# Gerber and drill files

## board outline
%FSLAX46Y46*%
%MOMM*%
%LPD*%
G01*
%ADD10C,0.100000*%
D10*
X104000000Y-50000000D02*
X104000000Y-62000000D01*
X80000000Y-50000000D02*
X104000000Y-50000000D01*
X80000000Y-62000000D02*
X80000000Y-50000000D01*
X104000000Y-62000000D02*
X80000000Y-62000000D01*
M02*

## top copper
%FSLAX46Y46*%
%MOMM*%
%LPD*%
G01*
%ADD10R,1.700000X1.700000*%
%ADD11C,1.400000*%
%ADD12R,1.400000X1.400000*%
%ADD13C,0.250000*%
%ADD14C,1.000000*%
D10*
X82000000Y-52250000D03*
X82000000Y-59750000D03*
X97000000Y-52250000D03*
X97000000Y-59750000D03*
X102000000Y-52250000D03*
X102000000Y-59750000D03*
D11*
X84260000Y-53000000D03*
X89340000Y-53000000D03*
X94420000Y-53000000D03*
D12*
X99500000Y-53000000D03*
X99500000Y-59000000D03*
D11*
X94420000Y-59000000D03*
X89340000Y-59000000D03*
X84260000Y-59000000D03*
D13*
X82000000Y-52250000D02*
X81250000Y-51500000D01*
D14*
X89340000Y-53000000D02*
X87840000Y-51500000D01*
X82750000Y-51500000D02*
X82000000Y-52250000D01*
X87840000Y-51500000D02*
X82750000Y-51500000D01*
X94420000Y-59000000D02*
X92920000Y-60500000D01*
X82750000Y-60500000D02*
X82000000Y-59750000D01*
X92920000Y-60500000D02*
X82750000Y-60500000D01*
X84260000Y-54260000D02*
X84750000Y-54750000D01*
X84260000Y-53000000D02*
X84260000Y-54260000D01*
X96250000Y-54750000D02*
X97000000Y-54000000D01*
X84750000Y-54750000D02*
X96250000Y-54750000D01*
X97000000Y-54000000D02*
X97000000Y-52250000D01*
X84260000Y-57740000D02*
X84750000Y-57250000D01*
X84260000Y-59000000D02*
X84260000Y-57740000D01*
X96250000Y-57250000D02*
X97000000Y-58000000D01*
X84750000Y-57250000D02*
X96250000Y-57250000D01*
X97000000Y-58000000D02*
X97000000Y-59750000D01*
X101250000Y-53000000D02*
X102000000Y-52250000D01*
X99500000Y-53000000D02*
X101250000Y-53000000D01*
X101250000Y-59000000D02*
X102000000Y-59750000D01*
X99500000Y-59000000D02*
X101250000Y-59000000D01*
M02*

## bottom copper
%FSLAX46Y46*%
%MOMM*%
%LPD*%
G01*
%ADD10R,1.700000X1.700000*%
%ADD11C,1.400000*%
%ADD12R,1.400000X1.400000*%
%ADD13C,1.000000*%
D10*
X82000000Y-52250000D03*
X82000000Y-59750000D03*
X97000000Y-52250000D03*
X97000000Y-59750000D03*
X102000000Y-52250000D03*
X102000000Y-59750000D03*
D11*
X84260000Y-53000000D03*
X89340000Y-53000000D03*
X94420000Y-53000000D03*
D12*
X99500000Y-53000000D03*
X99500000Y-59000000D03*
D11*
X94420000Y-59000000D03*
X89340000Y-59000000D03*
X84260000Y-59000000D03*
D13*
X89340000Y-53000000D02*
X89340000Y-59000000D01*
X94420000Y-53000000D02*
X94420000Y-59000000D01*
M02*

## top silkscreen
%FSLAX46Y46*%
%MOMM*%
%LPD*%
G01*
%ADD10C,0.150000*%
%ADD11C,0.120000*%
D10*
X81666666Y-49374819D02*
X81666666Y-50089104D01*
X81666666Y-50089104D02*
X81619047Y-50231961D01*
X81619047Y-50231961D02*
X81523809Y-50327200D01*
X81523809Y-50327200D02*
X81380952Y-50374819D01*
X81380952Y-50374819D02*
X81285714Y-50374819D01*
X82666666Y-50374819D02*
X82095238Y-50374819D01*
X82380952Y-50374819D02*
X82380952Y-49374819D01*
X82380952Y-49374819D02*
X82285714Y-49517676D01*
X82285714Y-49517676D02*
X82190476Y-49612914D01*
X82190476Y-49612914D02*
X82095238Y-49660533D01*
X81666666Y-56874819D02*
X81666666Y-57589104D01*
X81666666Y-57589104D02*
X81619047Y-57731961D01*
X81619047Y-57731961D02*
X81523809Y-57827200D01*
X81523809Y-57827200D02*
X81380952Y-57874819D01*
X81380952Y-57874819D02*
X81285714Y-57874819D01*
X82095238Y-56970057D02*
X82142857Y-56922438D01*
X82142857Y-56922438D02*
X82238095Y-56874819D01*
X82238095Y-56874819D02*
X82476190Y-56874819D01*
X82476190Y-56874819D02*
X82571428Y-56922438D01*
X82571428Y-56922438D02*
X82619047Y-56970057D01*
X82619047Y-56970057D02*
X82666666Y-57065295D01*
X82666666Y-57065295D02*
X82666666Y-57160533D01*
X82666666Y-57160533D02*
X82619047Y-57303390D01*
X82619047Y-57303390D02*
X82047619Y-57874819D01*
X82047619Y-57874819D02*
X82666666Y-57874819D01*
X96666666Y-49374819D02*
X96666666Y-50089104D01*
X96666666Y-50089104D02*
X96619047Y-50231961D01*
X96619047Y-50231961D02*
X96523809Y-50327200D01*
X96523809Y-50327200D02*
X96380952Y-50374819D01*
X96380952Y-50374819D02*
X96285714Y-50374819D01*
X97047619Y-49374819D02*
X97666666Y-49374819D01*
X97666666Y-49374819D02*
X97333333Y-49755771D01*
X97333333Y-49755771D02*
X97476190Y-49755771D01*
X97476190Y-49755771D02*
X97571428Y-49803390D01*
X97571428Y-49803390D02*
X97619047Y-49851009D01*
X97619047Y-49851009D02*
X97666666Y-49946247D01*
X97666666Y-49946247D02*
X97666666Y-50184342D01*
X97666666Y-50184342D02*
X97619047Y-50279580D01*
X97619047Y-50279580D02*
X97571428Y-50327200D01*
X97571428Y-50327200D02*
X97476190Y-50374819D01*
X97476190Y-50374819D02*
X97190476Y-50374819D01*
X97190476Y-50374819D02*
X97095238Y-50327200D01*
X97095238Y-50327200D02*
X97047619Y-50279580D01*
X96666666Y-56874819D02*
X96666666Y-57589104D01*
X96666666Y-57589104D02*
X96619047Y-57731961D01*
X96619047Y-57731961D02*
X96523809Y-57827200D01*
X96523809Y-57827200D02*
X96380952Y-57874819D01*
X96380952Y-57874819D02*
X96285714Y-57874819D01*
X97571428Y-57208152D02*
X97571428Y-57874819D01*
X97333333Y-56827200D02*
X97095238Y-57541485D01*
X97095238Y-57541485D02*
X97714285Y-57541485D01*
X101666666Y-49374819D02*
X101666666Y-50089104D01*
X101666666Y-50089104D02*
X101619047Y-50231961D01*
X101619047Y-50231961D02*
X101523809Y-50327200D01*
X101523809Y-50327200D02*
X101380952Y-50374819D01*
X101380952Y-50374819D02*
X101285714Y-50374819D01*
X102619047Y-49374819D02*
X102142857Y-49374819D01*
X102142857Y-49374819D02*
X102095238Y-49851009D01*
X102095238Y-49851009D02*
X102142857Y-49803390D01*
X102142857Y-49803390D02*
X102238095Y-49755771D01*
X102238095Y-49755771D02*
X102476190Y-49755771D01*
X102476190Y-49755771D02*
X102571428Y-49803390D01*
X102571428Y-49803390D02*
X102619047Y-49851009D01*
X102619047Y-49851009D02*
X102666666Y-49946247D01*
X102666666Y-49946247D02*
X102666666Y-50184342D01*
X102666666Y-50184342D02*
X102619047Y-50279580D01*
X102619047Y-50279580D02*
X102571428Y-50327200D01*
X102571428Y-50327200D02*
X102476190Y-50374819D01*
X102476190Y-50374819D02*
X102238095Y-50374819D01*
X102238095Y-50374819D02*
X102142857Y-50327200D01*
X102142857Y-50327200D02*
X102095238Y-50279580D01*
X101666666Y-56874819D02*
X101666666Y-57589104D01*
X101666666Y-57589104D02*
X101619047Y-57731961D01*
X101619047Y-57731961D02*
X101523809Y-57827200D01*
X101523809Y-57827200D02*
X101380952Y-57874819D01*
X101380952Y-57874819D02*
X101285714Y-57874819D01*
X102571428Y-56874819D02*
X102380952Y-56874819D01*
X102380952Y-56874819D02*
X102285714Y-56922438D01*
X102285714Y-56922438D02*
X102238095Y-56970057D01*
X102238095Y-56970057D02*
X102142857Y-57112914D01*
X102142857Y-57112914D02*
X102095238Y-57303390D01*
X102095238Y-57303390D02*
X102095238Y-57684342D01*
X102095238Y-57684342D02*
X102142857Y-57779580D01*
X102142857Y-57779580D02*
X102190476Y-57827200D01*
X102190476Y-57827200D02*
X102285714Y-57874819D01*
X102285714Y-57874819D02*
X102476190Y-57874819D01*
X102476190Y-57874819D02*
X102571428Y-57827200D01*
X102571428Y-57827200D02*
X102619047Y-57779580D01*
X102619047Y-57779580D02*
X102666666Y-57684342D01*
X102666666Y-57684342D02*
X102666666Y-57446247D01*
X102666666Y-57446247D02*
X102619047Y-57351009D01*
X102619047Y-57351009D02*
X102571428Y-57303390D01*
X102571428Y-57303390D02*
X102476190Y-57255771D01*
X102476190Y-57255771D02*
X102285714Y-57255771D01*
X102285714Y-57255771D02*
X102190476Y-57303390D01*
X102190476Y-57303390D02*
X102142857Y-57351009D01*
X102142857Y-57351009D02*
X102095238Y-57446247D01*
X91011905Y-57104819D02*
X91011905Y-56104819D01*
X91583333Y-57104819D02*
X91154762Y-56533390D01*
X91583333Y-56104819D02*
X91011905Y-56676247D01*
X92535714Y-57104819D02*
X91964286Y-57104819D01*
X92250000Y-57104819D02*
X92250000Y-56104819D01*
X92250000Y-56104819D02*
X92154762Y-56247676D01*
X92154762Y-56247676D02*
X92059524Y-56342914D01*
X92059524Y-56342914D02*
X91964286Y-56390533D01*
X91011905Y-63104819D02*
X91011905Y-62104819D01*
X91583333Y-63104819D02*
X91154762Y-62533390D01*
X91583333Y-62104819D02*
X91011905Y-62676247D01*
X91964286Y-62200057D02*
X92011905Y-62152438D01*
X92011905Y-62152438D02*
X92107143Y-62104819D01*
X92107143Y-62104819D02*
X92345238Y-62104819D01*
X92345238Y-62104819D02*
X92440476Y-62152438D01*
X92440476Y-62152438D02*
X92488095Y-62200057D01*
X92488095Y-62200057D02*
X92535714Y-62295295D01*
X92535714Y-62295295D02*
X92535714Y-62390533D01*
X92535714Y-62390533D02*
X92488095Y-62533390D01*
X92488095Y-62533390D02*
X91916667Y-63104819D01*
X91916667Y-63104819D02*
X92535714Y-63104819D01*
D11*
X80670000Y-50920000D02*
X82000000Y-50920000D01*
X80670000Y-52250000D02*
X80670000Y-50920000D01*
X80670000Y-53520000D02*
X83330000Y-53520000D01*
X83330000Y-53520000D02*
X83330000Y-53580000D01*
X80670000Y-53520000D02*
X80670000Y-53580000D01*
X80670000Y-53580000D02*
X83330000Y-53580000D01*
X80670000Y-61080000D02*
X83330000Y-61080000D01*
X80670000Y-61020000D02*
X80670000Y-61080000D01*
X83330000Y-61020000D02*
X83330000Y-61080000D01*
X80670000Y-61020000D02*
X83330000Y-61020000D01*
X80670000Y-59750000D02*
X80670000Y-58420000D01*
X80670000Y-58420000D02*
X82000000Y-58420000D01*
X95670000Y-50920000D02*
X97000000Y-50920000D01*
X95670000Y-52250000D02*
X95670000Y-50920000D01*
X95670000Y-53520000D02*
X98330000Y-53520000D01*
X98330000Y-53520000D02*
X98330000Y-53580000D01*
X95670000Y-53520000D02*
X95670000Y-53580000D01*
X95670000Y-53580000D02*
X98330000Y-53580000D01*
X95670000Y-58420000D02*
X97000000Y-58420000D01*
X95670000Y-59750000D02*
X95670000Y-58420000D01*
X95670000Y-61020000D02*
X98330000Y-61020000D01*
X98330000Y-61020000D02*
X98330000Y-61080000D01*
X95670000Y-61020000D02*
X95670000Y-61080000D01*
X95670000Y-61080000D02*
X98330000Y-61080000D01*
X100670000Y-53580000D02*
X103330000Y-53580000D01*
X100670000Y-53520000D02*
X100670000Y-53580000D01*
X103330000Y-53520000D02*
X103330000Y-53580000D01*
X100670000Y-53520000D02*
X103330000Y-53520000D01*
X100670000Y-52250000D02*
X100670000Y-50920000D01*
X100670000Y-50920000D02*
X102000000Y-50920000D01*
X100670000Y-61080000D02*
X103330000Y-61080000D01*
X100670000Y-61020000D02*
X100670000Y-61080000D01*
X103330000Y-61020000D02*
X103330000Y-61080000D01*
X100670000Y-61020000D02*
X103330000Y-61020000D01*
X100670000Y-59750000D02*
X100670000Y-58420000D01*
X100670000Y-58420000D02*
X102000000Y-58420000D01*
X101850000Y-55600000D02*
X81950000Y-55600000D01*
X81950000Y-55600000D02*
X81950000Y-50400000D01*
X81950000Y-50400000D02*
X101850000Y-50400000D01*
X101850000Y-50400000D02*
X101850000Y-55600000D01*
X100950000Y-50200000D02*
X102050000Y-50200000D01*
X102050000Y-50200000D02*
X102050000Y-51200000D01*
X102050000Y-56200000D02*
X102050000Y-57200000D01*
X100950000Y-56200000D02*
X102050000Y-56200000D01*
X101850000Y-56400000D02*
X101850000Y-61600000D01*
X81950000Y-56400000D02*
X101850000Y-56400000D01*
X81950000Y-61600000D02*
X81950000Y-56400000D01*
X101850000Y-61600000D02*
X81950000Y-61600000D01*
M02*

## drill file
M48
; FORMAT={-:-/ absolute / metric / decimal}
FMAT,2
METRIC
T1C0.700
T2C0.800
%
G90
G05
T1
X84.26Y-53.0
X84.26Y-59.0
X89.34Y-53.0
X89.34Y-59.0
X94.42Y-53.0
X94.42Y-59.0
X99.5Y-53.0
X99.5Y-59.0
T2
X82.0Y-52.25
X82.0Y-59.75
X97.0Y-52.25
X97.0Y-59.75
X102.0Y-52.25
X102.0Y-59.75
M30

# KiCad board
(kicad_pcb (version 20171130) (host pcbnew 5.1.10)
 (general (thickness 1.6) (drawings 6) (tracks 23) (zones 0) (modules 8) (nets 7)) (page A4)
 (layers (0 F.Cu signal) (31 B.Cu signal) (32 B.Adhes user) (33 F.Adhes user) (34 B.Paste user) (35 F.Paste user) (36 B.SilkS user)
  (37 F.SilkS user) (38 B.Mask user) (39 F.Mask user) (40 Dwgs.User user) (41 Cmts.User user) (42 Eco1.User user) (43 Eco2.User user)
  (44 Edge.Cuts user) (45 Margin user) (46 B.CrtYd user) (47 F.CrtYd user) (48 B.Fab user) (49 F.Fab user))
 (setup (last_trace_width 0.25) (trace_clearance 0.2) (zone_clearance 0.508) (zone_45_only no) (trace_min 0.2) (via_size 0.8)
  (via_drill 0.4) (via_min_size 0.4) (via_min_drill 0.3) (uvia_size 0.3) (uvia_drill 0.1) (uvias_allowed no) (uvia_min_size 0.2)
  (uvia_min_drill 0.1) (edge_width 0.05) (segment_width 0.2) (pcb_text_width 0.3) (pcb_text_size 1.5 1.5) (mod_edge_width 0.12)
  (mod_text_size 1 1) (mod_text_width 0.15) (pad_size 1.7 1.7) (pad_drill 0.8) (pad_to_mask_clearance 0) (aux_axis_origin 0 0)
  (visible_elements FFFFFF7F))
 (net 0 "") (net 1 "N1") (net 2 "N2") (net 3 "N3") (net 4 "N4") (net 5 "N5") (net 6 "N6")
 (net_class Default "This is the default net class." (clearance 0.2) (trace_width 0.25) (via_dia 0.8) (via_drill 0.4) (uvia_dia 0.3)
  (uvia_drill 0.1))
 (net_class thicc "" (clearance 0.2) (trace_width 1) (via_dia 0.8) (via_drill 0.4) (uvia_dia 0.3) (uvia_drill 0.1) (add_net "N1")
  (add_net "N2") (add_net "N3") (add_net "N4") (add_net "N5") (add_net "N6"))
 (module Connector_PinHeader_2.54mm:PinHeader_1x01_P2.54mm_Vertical (layer F.Cu) (at 82 52.25)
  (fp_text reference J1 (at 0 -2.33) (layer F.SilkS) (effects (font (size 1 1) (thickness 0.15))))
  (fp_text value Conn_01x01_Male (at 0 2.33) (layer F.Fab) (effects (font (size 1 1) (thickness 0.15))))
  (fp_line (start -1.33 -1.33) (end 0 -1.33) (layer F.SilkS) (width 0.12))
  (fp_line (start -1.33 0) (end -1.33 -1.33) (layer F.SilkS) (width 0.12))
  (fp_line (start -1.33 1.27) (end 1.33 1.27) (layer F.SilkS) (width 0.12))
  (fp_line (start 1.33 1.27) (end 1.33 1.33) (layer F.SilkS) (width 0.12))
  (fp_line (start -1.33 1.27) (end -1.33 1.33) (layer F.SilkS) (width 0.12))
  (fp_line (start -1.33 1.33) (end 1.33 1.33) (layer F.SilkS) (width 0.12))
  (pad 1 thru_hole rect (at 0 0) (size 1.7 1.7) (drill 0.8) (layers *.Cu *.Mask) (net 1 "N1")))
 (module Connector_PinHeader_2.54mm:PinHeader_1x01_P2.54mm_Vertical (layer F.Cu) (at 82 59.75)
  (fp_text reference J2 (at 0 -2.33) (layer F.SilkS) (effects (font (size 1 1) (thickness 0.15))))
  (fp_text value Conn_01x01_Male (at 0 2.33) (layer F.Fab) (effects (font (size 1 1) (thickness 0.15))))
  (fp_line (start -1.33 1.33) (end 1.33 1.33) (layer F.SilkS) (width 0.12))
  (fp_line (start -1.33 1.27) (end -1.33 1.33) (layer F.SilkS) (width 0.12))
  (fp_line (start 1.33 1.27) (end 1.33 1.33) (layer F.SilkS) (width 0.12))
  (fp_line (start -1.33 1.27) (end 1.33 1.27) (layer F.SilkS) (width 0.12))
  (fp_line (start -1.33 0) (end -1.33 -1.33) (layer F.SilkS) (width 0.12))
  (fp_line (start -1.33 -1.33) (end 0 -1.33) (layer F.SilkS) (width 0.12))
  (pad 1 thru_hole rect (at 0 0) (size 1.7 1.7) (drill 0.8) (layers *.Cu *.Mask) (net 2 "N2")))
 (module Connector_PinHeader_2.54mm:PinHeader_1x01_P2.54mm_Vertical (layer F.Cu) (at 97 52.25)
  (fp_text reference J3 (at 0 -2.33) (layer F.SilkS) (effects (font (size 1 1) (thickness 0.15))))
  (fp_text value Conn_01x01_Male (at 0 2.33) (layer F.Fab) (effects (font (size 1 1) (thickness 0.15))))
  (fp_line (start -1.33 -1.33) (end 0 -1.33) (layer F.SilkS) (width 0.12))
  (fp_line (start -1.33 0) (end -1.33 -1.33) (layer F.SilkS) (width 0.12))
  (fp_line (start -1.33 1.27) (end 1.33 1.27) (layer F.SilkS) (width 0.12))
  (fp_line (start 1.33 1.27) (end 1.33 1.33) (layer F.SilkS) (width 0.12))
  (fp_line (start -1.33 1.27) (end -1.33 1.33) (layer F.SilkS) (width 0.12))
  (fp_line (start -1.33 1.33) (end 1.33 1.33) (layer F.SilkS) (width 0.12))
  (pad 1 thru_hole rect (at 0 0) (size 1.7 1.7) (drill 0.8) (layers *.Cu *.Mask) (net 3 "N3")))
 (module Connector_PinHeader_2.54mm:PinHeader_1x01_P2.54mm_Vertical (layer F.Cu) (at 97 59.75)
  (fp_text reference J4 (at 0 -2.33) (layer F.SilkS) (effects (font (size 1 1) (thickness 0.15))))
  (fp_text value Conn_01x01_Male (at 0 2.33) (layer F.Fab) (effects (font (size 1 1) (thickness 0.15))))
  (fp_line (start -1.33 -1.33) (end 0 -1.33) (layer F.SilkS) (width 0.12))
  (fp_line (start -1.33 0) (end -1.33 -1.33) (layer F.SilkS) (width 0.12))
  (fp_line (start -1.33 1.27) (end 1.33 1.27) (layer F.SilkS) (width 0.12))
  (fp_line (start 1.33 1.27) (end 1.33 1.33) (layer F.SilkS) (width 0.12))
  (fp_line (start -1.33 1.27) (end -1.33 1.33) (layer F.SilkS) (width 0.12))
  (fp_line (start -1.33 1.33) (end 1.33 1.33) (layer F.SilkS) (width 0.12))
  (pad 1 thru_hole rect (at 0 0) (size 1.7 1.7) (drill 0.8) (layers *.Cu *.Mask) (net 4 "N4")))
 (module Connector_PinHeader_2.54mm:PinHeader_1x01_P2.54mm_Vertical (layer F.Cu) (at 102 52.25)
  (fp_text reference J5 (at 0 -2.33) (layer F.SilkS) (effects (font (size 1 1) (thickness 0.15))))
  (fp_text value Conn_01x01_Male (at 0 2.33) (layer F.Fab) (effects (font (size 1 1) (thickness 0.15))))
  (fp_line (start -1.33 1.33) (end 1.33 1.33) (layer F.SilkS) (width 0.12))
  (fp_line (start -1.33 1.27) (end -1.33 1.33) (layer F.SilkS) (width 0.12))
  (fp_line (start 1.33 1.27) (end 1.33 1.33) (layer F.SilkS) (width 0.12))
  (fp_line (start -1.33 1.27) (end 1.33 1.27) (layer F.SilkS) (width 0.12))
  (fp_line (start -1.33 0) (end -1.33 -1.33) (layer F.SilkS) (width 0.12))
  (fp_line (start -1.33 -1.33) (end 0 -1.33) (layer F.SilkS) (width 0.12))
  (pad 1 thru_hole rect (at 0 0) (size 1.7 1.7) (drill 0.8) (layers *.Cu *.Mask) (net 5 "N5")))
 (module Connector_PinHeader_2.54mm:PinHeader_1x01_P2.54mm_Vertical (layer F.Cu) (at 102 59.75)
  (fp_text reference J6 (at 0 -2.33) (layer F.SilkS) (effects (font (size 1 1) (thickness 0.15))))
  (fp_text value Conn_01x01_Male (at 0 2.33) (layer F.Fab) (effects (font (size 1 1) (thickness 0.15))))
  (fp_line (start -1.33 1.33) (end 1.33 1.33) (layer F.SilkS) (width 0.12))
  (fp_line (start -1.33 1.27) (end -1.33 1.33) (layer F.SilkS) (width 0.12))
  (fp_line (start 1.33 1.27) (end 1.33 1.33) (layer F.SilkS) (width 0.12))
  (fp_line (start -1.33 1.27) (end 1.33 1.27) (layer F.SilkS) (width 0.12))
  (fp_line (start -1.33 0) (end -1.33 -1.33) (layer F.SilkS) (width 0.12))
  (fp_line (start -1.33 -1.33) (end 0 -1.33) (layer F.SilkS) (width 0.12))
  (pad 1 thru_hole rect (at 0 0) (size 1.7 1.7) (drill 0.8) (layers *.Cu *.Mask) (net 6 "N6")))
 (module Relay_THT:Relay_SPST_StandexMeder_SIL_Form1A (layer F.Cu) (at 99.5 53 180)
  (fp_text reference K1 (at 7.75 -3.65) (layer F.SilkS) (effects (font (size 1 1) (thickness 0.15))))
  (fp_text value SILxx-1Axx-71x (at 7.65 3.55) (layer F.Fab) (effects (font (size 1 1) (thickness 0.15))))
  (fp_line (start -2.35 -2.6) (end 17.55 -2.6) (layer F.SilkS) (width 0.12))
  (fp_line (start 17.55 -2.6) (end 17.55 2.6) (layer F.SilkS) (width 0.12))
  (fp_line (start 17.55 2.6) (end -2.35 2.6) (layer F.SilkS) (width 0.12))
  (fp_line (start -2.35 2.6) (end -2.35 -2.6) (layer F.SilkS) (width 0.12))
  (fp_line (start -1.45 2.8) (end -2.55 2.8) (layer F.SilkS) (width 0.12))
  (fp_line (start -2.55 2.8) (end -2.55 1.8) (layer F.SilkS) (width 0.12))
  (pad 7 thru_hole circle (at 15.24 0 180) (size 1.4 1.4) (drill 0.7) (layers *.Cu *.Mask) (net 3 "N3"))
  (pad 5 thru_hole circle (at 10.16 0 180) (size 1.4 1.4) (drill 0.7) (layers *.Cu *.Mask) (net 1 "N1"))
  (pad 3 thru_hole circle (at 5.08 0 180) (size 1.4 1.4) (drill 0.7) (layers *.Cu *.Mask) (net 2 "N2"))
  (pad 1 thru_hole rect (at 0 0 180) (size 1.4 1.4) (drill 0.7) (layers *.Cu *.Mask) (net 5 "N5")))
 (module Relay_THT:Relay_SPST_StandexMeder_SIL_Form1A (layer F.Cu) (at 99.5 59 180)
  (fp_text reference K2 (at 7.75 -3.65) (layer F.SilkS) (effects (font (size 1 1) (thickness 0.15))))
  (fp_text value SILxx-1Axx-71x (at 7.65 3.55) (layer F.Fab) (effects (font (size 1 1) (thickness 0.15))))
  (fp_line (start -2.55 2.8) (end -2.55 1.8) (layer F.SilkS) (width 0.12))
  (fp_line (start -1.45 2.8) (end -2.55 2.8) (layer F.SilkS) (width 0.12))
  (fp_line (start -2.35 2.6) (end -2.35 -2.6) (layer F.SilkS) (width 0.12))
  (fp_line (start 17.55 2.6) (end -2.35 2.6) (layer F.SilkS) (width 0.12))
  (fp_line (start 17.55 -2.6) (end 17.55 2.6) (layer F.SilkS) (width 0.12))
  (fp_line (start -2.35 -2.6) (end 17.55 -2.6) (layer F.SilkS) (width 0.12))
  (pad 1 thru_hole rect (at 0 0 180) (size 1.4 1.4) (drill 0.7) (layers *.Cu *.Mask) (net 6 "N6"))
  (pad 3 thru_hole circle (at 5.08 0 180) (size 1.4 1.4) (drill 0.7) (layers *.Cu *.Mask) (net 2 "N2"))
  (pad 5 thru_hole circle (at 10.16 0 180) (size 1.4 1.4) (drill 0.7) (layers *.Cu *.Mask) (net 1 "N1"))
  (pad 7 thru_hole circle (at 15.24 0 180) (size 1.4 1.4) (drill 0.7) (layers *.Cu *.Mask) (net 4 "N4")))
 (gr_line (start 104 50) (end 104 62) (layer Edge.Cuts) (width 0.1))
 (gr_line (start 80 50) (end 104 50) (layer Edge.Cuts) (width 0.1))
 (gr_line (start 80 62) (end 80 50) (layer Edge.Cuts) (width 0.1))
 (gr_line (start 104 62) (end 80 62) (layer Edge.Cuts) (width 0.1))
 (segment (start 82 52.25) (end 81.25 51.5) (width 0.25) (layer F.Cu) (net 1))
 (segment (start 89.34 53) (end 89.34 59) (width 1) (layer B.Cu) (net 1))
 (segment (start 89.34 53) (end 87.84 51.5) (width 1) (layer F.Cu) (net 1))
 (segment (start 82.75 51.5) (end 82 52.25) (width 1) (layer F.Cu) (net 1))
 (segment (start 87.84 51.5) (end 82.75 51.5) (width 1) (layer F.Cu) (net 1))
 (segment (start 94.42 53) (end 94.42 59) (width 1) (layer B.Cu) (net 2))
 (segment (start 94.42 59) (end 92.92 60.5) (width 1) (layer F.Cu) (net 2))
 (segment (start 82.75 60.5) (end 82 59.75) (width 1) (layer F.Cu) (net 2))
 (segment (start 92.92 60.5) (end 82.75 60.5) (width 1) (layer F.Cu) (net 2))
 (segment (start 84.26 54.26) (end 84.75 54.75) (width 1) (layer F.Cu) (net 3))
 (segment (start 84.26 53) (end 84.26 54.26) (width 1) (layer F.Cu) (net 3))
 (segment (start 96.25 54.75) (end 97 54) (width 1) (layer F.Cu) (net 3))
 (segment (start 84.75 54.75) (end 96.25 54.75) (width 1) (layer F.Cu) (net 3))
 (segment (start 97 54) (end 97 52.25) (width 1) (layer F.Cu) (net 3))
 (segment (start 84.26 57.74) (end 84.75 57.25) (width 1) (layer F.Cu) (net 4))
 (segment (start 84.26 59) (end 84.26 57.74) (width 1) (layer F.Cu) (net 4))
 (segment (start 96.25 57.25) (end 97 58) (width 1) (layer F.Cu) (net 4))
 (segment (start 84.75 57.25) (end 96.25 57.25) (width 1) (layer F.Cu) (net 4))
 (segment (start 97 58) (end 97 59.75) (width 1) (layer F.Cu) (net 4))
 (segment (start 101.25 53) (end 102 52.25) (width 1) (layer F.Cu) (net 5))
 (segment (start 99.5 53) (end 101.25 53) (width 1) (layer F.Cu) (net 5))
 (segment (start 101.25 59) (end 102 59.75) (width 1) (layer F.Cu) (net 6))
 (segment (start 99.5 59) (end 101.25 59) (width 1) (layer F.Cu) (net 6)))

